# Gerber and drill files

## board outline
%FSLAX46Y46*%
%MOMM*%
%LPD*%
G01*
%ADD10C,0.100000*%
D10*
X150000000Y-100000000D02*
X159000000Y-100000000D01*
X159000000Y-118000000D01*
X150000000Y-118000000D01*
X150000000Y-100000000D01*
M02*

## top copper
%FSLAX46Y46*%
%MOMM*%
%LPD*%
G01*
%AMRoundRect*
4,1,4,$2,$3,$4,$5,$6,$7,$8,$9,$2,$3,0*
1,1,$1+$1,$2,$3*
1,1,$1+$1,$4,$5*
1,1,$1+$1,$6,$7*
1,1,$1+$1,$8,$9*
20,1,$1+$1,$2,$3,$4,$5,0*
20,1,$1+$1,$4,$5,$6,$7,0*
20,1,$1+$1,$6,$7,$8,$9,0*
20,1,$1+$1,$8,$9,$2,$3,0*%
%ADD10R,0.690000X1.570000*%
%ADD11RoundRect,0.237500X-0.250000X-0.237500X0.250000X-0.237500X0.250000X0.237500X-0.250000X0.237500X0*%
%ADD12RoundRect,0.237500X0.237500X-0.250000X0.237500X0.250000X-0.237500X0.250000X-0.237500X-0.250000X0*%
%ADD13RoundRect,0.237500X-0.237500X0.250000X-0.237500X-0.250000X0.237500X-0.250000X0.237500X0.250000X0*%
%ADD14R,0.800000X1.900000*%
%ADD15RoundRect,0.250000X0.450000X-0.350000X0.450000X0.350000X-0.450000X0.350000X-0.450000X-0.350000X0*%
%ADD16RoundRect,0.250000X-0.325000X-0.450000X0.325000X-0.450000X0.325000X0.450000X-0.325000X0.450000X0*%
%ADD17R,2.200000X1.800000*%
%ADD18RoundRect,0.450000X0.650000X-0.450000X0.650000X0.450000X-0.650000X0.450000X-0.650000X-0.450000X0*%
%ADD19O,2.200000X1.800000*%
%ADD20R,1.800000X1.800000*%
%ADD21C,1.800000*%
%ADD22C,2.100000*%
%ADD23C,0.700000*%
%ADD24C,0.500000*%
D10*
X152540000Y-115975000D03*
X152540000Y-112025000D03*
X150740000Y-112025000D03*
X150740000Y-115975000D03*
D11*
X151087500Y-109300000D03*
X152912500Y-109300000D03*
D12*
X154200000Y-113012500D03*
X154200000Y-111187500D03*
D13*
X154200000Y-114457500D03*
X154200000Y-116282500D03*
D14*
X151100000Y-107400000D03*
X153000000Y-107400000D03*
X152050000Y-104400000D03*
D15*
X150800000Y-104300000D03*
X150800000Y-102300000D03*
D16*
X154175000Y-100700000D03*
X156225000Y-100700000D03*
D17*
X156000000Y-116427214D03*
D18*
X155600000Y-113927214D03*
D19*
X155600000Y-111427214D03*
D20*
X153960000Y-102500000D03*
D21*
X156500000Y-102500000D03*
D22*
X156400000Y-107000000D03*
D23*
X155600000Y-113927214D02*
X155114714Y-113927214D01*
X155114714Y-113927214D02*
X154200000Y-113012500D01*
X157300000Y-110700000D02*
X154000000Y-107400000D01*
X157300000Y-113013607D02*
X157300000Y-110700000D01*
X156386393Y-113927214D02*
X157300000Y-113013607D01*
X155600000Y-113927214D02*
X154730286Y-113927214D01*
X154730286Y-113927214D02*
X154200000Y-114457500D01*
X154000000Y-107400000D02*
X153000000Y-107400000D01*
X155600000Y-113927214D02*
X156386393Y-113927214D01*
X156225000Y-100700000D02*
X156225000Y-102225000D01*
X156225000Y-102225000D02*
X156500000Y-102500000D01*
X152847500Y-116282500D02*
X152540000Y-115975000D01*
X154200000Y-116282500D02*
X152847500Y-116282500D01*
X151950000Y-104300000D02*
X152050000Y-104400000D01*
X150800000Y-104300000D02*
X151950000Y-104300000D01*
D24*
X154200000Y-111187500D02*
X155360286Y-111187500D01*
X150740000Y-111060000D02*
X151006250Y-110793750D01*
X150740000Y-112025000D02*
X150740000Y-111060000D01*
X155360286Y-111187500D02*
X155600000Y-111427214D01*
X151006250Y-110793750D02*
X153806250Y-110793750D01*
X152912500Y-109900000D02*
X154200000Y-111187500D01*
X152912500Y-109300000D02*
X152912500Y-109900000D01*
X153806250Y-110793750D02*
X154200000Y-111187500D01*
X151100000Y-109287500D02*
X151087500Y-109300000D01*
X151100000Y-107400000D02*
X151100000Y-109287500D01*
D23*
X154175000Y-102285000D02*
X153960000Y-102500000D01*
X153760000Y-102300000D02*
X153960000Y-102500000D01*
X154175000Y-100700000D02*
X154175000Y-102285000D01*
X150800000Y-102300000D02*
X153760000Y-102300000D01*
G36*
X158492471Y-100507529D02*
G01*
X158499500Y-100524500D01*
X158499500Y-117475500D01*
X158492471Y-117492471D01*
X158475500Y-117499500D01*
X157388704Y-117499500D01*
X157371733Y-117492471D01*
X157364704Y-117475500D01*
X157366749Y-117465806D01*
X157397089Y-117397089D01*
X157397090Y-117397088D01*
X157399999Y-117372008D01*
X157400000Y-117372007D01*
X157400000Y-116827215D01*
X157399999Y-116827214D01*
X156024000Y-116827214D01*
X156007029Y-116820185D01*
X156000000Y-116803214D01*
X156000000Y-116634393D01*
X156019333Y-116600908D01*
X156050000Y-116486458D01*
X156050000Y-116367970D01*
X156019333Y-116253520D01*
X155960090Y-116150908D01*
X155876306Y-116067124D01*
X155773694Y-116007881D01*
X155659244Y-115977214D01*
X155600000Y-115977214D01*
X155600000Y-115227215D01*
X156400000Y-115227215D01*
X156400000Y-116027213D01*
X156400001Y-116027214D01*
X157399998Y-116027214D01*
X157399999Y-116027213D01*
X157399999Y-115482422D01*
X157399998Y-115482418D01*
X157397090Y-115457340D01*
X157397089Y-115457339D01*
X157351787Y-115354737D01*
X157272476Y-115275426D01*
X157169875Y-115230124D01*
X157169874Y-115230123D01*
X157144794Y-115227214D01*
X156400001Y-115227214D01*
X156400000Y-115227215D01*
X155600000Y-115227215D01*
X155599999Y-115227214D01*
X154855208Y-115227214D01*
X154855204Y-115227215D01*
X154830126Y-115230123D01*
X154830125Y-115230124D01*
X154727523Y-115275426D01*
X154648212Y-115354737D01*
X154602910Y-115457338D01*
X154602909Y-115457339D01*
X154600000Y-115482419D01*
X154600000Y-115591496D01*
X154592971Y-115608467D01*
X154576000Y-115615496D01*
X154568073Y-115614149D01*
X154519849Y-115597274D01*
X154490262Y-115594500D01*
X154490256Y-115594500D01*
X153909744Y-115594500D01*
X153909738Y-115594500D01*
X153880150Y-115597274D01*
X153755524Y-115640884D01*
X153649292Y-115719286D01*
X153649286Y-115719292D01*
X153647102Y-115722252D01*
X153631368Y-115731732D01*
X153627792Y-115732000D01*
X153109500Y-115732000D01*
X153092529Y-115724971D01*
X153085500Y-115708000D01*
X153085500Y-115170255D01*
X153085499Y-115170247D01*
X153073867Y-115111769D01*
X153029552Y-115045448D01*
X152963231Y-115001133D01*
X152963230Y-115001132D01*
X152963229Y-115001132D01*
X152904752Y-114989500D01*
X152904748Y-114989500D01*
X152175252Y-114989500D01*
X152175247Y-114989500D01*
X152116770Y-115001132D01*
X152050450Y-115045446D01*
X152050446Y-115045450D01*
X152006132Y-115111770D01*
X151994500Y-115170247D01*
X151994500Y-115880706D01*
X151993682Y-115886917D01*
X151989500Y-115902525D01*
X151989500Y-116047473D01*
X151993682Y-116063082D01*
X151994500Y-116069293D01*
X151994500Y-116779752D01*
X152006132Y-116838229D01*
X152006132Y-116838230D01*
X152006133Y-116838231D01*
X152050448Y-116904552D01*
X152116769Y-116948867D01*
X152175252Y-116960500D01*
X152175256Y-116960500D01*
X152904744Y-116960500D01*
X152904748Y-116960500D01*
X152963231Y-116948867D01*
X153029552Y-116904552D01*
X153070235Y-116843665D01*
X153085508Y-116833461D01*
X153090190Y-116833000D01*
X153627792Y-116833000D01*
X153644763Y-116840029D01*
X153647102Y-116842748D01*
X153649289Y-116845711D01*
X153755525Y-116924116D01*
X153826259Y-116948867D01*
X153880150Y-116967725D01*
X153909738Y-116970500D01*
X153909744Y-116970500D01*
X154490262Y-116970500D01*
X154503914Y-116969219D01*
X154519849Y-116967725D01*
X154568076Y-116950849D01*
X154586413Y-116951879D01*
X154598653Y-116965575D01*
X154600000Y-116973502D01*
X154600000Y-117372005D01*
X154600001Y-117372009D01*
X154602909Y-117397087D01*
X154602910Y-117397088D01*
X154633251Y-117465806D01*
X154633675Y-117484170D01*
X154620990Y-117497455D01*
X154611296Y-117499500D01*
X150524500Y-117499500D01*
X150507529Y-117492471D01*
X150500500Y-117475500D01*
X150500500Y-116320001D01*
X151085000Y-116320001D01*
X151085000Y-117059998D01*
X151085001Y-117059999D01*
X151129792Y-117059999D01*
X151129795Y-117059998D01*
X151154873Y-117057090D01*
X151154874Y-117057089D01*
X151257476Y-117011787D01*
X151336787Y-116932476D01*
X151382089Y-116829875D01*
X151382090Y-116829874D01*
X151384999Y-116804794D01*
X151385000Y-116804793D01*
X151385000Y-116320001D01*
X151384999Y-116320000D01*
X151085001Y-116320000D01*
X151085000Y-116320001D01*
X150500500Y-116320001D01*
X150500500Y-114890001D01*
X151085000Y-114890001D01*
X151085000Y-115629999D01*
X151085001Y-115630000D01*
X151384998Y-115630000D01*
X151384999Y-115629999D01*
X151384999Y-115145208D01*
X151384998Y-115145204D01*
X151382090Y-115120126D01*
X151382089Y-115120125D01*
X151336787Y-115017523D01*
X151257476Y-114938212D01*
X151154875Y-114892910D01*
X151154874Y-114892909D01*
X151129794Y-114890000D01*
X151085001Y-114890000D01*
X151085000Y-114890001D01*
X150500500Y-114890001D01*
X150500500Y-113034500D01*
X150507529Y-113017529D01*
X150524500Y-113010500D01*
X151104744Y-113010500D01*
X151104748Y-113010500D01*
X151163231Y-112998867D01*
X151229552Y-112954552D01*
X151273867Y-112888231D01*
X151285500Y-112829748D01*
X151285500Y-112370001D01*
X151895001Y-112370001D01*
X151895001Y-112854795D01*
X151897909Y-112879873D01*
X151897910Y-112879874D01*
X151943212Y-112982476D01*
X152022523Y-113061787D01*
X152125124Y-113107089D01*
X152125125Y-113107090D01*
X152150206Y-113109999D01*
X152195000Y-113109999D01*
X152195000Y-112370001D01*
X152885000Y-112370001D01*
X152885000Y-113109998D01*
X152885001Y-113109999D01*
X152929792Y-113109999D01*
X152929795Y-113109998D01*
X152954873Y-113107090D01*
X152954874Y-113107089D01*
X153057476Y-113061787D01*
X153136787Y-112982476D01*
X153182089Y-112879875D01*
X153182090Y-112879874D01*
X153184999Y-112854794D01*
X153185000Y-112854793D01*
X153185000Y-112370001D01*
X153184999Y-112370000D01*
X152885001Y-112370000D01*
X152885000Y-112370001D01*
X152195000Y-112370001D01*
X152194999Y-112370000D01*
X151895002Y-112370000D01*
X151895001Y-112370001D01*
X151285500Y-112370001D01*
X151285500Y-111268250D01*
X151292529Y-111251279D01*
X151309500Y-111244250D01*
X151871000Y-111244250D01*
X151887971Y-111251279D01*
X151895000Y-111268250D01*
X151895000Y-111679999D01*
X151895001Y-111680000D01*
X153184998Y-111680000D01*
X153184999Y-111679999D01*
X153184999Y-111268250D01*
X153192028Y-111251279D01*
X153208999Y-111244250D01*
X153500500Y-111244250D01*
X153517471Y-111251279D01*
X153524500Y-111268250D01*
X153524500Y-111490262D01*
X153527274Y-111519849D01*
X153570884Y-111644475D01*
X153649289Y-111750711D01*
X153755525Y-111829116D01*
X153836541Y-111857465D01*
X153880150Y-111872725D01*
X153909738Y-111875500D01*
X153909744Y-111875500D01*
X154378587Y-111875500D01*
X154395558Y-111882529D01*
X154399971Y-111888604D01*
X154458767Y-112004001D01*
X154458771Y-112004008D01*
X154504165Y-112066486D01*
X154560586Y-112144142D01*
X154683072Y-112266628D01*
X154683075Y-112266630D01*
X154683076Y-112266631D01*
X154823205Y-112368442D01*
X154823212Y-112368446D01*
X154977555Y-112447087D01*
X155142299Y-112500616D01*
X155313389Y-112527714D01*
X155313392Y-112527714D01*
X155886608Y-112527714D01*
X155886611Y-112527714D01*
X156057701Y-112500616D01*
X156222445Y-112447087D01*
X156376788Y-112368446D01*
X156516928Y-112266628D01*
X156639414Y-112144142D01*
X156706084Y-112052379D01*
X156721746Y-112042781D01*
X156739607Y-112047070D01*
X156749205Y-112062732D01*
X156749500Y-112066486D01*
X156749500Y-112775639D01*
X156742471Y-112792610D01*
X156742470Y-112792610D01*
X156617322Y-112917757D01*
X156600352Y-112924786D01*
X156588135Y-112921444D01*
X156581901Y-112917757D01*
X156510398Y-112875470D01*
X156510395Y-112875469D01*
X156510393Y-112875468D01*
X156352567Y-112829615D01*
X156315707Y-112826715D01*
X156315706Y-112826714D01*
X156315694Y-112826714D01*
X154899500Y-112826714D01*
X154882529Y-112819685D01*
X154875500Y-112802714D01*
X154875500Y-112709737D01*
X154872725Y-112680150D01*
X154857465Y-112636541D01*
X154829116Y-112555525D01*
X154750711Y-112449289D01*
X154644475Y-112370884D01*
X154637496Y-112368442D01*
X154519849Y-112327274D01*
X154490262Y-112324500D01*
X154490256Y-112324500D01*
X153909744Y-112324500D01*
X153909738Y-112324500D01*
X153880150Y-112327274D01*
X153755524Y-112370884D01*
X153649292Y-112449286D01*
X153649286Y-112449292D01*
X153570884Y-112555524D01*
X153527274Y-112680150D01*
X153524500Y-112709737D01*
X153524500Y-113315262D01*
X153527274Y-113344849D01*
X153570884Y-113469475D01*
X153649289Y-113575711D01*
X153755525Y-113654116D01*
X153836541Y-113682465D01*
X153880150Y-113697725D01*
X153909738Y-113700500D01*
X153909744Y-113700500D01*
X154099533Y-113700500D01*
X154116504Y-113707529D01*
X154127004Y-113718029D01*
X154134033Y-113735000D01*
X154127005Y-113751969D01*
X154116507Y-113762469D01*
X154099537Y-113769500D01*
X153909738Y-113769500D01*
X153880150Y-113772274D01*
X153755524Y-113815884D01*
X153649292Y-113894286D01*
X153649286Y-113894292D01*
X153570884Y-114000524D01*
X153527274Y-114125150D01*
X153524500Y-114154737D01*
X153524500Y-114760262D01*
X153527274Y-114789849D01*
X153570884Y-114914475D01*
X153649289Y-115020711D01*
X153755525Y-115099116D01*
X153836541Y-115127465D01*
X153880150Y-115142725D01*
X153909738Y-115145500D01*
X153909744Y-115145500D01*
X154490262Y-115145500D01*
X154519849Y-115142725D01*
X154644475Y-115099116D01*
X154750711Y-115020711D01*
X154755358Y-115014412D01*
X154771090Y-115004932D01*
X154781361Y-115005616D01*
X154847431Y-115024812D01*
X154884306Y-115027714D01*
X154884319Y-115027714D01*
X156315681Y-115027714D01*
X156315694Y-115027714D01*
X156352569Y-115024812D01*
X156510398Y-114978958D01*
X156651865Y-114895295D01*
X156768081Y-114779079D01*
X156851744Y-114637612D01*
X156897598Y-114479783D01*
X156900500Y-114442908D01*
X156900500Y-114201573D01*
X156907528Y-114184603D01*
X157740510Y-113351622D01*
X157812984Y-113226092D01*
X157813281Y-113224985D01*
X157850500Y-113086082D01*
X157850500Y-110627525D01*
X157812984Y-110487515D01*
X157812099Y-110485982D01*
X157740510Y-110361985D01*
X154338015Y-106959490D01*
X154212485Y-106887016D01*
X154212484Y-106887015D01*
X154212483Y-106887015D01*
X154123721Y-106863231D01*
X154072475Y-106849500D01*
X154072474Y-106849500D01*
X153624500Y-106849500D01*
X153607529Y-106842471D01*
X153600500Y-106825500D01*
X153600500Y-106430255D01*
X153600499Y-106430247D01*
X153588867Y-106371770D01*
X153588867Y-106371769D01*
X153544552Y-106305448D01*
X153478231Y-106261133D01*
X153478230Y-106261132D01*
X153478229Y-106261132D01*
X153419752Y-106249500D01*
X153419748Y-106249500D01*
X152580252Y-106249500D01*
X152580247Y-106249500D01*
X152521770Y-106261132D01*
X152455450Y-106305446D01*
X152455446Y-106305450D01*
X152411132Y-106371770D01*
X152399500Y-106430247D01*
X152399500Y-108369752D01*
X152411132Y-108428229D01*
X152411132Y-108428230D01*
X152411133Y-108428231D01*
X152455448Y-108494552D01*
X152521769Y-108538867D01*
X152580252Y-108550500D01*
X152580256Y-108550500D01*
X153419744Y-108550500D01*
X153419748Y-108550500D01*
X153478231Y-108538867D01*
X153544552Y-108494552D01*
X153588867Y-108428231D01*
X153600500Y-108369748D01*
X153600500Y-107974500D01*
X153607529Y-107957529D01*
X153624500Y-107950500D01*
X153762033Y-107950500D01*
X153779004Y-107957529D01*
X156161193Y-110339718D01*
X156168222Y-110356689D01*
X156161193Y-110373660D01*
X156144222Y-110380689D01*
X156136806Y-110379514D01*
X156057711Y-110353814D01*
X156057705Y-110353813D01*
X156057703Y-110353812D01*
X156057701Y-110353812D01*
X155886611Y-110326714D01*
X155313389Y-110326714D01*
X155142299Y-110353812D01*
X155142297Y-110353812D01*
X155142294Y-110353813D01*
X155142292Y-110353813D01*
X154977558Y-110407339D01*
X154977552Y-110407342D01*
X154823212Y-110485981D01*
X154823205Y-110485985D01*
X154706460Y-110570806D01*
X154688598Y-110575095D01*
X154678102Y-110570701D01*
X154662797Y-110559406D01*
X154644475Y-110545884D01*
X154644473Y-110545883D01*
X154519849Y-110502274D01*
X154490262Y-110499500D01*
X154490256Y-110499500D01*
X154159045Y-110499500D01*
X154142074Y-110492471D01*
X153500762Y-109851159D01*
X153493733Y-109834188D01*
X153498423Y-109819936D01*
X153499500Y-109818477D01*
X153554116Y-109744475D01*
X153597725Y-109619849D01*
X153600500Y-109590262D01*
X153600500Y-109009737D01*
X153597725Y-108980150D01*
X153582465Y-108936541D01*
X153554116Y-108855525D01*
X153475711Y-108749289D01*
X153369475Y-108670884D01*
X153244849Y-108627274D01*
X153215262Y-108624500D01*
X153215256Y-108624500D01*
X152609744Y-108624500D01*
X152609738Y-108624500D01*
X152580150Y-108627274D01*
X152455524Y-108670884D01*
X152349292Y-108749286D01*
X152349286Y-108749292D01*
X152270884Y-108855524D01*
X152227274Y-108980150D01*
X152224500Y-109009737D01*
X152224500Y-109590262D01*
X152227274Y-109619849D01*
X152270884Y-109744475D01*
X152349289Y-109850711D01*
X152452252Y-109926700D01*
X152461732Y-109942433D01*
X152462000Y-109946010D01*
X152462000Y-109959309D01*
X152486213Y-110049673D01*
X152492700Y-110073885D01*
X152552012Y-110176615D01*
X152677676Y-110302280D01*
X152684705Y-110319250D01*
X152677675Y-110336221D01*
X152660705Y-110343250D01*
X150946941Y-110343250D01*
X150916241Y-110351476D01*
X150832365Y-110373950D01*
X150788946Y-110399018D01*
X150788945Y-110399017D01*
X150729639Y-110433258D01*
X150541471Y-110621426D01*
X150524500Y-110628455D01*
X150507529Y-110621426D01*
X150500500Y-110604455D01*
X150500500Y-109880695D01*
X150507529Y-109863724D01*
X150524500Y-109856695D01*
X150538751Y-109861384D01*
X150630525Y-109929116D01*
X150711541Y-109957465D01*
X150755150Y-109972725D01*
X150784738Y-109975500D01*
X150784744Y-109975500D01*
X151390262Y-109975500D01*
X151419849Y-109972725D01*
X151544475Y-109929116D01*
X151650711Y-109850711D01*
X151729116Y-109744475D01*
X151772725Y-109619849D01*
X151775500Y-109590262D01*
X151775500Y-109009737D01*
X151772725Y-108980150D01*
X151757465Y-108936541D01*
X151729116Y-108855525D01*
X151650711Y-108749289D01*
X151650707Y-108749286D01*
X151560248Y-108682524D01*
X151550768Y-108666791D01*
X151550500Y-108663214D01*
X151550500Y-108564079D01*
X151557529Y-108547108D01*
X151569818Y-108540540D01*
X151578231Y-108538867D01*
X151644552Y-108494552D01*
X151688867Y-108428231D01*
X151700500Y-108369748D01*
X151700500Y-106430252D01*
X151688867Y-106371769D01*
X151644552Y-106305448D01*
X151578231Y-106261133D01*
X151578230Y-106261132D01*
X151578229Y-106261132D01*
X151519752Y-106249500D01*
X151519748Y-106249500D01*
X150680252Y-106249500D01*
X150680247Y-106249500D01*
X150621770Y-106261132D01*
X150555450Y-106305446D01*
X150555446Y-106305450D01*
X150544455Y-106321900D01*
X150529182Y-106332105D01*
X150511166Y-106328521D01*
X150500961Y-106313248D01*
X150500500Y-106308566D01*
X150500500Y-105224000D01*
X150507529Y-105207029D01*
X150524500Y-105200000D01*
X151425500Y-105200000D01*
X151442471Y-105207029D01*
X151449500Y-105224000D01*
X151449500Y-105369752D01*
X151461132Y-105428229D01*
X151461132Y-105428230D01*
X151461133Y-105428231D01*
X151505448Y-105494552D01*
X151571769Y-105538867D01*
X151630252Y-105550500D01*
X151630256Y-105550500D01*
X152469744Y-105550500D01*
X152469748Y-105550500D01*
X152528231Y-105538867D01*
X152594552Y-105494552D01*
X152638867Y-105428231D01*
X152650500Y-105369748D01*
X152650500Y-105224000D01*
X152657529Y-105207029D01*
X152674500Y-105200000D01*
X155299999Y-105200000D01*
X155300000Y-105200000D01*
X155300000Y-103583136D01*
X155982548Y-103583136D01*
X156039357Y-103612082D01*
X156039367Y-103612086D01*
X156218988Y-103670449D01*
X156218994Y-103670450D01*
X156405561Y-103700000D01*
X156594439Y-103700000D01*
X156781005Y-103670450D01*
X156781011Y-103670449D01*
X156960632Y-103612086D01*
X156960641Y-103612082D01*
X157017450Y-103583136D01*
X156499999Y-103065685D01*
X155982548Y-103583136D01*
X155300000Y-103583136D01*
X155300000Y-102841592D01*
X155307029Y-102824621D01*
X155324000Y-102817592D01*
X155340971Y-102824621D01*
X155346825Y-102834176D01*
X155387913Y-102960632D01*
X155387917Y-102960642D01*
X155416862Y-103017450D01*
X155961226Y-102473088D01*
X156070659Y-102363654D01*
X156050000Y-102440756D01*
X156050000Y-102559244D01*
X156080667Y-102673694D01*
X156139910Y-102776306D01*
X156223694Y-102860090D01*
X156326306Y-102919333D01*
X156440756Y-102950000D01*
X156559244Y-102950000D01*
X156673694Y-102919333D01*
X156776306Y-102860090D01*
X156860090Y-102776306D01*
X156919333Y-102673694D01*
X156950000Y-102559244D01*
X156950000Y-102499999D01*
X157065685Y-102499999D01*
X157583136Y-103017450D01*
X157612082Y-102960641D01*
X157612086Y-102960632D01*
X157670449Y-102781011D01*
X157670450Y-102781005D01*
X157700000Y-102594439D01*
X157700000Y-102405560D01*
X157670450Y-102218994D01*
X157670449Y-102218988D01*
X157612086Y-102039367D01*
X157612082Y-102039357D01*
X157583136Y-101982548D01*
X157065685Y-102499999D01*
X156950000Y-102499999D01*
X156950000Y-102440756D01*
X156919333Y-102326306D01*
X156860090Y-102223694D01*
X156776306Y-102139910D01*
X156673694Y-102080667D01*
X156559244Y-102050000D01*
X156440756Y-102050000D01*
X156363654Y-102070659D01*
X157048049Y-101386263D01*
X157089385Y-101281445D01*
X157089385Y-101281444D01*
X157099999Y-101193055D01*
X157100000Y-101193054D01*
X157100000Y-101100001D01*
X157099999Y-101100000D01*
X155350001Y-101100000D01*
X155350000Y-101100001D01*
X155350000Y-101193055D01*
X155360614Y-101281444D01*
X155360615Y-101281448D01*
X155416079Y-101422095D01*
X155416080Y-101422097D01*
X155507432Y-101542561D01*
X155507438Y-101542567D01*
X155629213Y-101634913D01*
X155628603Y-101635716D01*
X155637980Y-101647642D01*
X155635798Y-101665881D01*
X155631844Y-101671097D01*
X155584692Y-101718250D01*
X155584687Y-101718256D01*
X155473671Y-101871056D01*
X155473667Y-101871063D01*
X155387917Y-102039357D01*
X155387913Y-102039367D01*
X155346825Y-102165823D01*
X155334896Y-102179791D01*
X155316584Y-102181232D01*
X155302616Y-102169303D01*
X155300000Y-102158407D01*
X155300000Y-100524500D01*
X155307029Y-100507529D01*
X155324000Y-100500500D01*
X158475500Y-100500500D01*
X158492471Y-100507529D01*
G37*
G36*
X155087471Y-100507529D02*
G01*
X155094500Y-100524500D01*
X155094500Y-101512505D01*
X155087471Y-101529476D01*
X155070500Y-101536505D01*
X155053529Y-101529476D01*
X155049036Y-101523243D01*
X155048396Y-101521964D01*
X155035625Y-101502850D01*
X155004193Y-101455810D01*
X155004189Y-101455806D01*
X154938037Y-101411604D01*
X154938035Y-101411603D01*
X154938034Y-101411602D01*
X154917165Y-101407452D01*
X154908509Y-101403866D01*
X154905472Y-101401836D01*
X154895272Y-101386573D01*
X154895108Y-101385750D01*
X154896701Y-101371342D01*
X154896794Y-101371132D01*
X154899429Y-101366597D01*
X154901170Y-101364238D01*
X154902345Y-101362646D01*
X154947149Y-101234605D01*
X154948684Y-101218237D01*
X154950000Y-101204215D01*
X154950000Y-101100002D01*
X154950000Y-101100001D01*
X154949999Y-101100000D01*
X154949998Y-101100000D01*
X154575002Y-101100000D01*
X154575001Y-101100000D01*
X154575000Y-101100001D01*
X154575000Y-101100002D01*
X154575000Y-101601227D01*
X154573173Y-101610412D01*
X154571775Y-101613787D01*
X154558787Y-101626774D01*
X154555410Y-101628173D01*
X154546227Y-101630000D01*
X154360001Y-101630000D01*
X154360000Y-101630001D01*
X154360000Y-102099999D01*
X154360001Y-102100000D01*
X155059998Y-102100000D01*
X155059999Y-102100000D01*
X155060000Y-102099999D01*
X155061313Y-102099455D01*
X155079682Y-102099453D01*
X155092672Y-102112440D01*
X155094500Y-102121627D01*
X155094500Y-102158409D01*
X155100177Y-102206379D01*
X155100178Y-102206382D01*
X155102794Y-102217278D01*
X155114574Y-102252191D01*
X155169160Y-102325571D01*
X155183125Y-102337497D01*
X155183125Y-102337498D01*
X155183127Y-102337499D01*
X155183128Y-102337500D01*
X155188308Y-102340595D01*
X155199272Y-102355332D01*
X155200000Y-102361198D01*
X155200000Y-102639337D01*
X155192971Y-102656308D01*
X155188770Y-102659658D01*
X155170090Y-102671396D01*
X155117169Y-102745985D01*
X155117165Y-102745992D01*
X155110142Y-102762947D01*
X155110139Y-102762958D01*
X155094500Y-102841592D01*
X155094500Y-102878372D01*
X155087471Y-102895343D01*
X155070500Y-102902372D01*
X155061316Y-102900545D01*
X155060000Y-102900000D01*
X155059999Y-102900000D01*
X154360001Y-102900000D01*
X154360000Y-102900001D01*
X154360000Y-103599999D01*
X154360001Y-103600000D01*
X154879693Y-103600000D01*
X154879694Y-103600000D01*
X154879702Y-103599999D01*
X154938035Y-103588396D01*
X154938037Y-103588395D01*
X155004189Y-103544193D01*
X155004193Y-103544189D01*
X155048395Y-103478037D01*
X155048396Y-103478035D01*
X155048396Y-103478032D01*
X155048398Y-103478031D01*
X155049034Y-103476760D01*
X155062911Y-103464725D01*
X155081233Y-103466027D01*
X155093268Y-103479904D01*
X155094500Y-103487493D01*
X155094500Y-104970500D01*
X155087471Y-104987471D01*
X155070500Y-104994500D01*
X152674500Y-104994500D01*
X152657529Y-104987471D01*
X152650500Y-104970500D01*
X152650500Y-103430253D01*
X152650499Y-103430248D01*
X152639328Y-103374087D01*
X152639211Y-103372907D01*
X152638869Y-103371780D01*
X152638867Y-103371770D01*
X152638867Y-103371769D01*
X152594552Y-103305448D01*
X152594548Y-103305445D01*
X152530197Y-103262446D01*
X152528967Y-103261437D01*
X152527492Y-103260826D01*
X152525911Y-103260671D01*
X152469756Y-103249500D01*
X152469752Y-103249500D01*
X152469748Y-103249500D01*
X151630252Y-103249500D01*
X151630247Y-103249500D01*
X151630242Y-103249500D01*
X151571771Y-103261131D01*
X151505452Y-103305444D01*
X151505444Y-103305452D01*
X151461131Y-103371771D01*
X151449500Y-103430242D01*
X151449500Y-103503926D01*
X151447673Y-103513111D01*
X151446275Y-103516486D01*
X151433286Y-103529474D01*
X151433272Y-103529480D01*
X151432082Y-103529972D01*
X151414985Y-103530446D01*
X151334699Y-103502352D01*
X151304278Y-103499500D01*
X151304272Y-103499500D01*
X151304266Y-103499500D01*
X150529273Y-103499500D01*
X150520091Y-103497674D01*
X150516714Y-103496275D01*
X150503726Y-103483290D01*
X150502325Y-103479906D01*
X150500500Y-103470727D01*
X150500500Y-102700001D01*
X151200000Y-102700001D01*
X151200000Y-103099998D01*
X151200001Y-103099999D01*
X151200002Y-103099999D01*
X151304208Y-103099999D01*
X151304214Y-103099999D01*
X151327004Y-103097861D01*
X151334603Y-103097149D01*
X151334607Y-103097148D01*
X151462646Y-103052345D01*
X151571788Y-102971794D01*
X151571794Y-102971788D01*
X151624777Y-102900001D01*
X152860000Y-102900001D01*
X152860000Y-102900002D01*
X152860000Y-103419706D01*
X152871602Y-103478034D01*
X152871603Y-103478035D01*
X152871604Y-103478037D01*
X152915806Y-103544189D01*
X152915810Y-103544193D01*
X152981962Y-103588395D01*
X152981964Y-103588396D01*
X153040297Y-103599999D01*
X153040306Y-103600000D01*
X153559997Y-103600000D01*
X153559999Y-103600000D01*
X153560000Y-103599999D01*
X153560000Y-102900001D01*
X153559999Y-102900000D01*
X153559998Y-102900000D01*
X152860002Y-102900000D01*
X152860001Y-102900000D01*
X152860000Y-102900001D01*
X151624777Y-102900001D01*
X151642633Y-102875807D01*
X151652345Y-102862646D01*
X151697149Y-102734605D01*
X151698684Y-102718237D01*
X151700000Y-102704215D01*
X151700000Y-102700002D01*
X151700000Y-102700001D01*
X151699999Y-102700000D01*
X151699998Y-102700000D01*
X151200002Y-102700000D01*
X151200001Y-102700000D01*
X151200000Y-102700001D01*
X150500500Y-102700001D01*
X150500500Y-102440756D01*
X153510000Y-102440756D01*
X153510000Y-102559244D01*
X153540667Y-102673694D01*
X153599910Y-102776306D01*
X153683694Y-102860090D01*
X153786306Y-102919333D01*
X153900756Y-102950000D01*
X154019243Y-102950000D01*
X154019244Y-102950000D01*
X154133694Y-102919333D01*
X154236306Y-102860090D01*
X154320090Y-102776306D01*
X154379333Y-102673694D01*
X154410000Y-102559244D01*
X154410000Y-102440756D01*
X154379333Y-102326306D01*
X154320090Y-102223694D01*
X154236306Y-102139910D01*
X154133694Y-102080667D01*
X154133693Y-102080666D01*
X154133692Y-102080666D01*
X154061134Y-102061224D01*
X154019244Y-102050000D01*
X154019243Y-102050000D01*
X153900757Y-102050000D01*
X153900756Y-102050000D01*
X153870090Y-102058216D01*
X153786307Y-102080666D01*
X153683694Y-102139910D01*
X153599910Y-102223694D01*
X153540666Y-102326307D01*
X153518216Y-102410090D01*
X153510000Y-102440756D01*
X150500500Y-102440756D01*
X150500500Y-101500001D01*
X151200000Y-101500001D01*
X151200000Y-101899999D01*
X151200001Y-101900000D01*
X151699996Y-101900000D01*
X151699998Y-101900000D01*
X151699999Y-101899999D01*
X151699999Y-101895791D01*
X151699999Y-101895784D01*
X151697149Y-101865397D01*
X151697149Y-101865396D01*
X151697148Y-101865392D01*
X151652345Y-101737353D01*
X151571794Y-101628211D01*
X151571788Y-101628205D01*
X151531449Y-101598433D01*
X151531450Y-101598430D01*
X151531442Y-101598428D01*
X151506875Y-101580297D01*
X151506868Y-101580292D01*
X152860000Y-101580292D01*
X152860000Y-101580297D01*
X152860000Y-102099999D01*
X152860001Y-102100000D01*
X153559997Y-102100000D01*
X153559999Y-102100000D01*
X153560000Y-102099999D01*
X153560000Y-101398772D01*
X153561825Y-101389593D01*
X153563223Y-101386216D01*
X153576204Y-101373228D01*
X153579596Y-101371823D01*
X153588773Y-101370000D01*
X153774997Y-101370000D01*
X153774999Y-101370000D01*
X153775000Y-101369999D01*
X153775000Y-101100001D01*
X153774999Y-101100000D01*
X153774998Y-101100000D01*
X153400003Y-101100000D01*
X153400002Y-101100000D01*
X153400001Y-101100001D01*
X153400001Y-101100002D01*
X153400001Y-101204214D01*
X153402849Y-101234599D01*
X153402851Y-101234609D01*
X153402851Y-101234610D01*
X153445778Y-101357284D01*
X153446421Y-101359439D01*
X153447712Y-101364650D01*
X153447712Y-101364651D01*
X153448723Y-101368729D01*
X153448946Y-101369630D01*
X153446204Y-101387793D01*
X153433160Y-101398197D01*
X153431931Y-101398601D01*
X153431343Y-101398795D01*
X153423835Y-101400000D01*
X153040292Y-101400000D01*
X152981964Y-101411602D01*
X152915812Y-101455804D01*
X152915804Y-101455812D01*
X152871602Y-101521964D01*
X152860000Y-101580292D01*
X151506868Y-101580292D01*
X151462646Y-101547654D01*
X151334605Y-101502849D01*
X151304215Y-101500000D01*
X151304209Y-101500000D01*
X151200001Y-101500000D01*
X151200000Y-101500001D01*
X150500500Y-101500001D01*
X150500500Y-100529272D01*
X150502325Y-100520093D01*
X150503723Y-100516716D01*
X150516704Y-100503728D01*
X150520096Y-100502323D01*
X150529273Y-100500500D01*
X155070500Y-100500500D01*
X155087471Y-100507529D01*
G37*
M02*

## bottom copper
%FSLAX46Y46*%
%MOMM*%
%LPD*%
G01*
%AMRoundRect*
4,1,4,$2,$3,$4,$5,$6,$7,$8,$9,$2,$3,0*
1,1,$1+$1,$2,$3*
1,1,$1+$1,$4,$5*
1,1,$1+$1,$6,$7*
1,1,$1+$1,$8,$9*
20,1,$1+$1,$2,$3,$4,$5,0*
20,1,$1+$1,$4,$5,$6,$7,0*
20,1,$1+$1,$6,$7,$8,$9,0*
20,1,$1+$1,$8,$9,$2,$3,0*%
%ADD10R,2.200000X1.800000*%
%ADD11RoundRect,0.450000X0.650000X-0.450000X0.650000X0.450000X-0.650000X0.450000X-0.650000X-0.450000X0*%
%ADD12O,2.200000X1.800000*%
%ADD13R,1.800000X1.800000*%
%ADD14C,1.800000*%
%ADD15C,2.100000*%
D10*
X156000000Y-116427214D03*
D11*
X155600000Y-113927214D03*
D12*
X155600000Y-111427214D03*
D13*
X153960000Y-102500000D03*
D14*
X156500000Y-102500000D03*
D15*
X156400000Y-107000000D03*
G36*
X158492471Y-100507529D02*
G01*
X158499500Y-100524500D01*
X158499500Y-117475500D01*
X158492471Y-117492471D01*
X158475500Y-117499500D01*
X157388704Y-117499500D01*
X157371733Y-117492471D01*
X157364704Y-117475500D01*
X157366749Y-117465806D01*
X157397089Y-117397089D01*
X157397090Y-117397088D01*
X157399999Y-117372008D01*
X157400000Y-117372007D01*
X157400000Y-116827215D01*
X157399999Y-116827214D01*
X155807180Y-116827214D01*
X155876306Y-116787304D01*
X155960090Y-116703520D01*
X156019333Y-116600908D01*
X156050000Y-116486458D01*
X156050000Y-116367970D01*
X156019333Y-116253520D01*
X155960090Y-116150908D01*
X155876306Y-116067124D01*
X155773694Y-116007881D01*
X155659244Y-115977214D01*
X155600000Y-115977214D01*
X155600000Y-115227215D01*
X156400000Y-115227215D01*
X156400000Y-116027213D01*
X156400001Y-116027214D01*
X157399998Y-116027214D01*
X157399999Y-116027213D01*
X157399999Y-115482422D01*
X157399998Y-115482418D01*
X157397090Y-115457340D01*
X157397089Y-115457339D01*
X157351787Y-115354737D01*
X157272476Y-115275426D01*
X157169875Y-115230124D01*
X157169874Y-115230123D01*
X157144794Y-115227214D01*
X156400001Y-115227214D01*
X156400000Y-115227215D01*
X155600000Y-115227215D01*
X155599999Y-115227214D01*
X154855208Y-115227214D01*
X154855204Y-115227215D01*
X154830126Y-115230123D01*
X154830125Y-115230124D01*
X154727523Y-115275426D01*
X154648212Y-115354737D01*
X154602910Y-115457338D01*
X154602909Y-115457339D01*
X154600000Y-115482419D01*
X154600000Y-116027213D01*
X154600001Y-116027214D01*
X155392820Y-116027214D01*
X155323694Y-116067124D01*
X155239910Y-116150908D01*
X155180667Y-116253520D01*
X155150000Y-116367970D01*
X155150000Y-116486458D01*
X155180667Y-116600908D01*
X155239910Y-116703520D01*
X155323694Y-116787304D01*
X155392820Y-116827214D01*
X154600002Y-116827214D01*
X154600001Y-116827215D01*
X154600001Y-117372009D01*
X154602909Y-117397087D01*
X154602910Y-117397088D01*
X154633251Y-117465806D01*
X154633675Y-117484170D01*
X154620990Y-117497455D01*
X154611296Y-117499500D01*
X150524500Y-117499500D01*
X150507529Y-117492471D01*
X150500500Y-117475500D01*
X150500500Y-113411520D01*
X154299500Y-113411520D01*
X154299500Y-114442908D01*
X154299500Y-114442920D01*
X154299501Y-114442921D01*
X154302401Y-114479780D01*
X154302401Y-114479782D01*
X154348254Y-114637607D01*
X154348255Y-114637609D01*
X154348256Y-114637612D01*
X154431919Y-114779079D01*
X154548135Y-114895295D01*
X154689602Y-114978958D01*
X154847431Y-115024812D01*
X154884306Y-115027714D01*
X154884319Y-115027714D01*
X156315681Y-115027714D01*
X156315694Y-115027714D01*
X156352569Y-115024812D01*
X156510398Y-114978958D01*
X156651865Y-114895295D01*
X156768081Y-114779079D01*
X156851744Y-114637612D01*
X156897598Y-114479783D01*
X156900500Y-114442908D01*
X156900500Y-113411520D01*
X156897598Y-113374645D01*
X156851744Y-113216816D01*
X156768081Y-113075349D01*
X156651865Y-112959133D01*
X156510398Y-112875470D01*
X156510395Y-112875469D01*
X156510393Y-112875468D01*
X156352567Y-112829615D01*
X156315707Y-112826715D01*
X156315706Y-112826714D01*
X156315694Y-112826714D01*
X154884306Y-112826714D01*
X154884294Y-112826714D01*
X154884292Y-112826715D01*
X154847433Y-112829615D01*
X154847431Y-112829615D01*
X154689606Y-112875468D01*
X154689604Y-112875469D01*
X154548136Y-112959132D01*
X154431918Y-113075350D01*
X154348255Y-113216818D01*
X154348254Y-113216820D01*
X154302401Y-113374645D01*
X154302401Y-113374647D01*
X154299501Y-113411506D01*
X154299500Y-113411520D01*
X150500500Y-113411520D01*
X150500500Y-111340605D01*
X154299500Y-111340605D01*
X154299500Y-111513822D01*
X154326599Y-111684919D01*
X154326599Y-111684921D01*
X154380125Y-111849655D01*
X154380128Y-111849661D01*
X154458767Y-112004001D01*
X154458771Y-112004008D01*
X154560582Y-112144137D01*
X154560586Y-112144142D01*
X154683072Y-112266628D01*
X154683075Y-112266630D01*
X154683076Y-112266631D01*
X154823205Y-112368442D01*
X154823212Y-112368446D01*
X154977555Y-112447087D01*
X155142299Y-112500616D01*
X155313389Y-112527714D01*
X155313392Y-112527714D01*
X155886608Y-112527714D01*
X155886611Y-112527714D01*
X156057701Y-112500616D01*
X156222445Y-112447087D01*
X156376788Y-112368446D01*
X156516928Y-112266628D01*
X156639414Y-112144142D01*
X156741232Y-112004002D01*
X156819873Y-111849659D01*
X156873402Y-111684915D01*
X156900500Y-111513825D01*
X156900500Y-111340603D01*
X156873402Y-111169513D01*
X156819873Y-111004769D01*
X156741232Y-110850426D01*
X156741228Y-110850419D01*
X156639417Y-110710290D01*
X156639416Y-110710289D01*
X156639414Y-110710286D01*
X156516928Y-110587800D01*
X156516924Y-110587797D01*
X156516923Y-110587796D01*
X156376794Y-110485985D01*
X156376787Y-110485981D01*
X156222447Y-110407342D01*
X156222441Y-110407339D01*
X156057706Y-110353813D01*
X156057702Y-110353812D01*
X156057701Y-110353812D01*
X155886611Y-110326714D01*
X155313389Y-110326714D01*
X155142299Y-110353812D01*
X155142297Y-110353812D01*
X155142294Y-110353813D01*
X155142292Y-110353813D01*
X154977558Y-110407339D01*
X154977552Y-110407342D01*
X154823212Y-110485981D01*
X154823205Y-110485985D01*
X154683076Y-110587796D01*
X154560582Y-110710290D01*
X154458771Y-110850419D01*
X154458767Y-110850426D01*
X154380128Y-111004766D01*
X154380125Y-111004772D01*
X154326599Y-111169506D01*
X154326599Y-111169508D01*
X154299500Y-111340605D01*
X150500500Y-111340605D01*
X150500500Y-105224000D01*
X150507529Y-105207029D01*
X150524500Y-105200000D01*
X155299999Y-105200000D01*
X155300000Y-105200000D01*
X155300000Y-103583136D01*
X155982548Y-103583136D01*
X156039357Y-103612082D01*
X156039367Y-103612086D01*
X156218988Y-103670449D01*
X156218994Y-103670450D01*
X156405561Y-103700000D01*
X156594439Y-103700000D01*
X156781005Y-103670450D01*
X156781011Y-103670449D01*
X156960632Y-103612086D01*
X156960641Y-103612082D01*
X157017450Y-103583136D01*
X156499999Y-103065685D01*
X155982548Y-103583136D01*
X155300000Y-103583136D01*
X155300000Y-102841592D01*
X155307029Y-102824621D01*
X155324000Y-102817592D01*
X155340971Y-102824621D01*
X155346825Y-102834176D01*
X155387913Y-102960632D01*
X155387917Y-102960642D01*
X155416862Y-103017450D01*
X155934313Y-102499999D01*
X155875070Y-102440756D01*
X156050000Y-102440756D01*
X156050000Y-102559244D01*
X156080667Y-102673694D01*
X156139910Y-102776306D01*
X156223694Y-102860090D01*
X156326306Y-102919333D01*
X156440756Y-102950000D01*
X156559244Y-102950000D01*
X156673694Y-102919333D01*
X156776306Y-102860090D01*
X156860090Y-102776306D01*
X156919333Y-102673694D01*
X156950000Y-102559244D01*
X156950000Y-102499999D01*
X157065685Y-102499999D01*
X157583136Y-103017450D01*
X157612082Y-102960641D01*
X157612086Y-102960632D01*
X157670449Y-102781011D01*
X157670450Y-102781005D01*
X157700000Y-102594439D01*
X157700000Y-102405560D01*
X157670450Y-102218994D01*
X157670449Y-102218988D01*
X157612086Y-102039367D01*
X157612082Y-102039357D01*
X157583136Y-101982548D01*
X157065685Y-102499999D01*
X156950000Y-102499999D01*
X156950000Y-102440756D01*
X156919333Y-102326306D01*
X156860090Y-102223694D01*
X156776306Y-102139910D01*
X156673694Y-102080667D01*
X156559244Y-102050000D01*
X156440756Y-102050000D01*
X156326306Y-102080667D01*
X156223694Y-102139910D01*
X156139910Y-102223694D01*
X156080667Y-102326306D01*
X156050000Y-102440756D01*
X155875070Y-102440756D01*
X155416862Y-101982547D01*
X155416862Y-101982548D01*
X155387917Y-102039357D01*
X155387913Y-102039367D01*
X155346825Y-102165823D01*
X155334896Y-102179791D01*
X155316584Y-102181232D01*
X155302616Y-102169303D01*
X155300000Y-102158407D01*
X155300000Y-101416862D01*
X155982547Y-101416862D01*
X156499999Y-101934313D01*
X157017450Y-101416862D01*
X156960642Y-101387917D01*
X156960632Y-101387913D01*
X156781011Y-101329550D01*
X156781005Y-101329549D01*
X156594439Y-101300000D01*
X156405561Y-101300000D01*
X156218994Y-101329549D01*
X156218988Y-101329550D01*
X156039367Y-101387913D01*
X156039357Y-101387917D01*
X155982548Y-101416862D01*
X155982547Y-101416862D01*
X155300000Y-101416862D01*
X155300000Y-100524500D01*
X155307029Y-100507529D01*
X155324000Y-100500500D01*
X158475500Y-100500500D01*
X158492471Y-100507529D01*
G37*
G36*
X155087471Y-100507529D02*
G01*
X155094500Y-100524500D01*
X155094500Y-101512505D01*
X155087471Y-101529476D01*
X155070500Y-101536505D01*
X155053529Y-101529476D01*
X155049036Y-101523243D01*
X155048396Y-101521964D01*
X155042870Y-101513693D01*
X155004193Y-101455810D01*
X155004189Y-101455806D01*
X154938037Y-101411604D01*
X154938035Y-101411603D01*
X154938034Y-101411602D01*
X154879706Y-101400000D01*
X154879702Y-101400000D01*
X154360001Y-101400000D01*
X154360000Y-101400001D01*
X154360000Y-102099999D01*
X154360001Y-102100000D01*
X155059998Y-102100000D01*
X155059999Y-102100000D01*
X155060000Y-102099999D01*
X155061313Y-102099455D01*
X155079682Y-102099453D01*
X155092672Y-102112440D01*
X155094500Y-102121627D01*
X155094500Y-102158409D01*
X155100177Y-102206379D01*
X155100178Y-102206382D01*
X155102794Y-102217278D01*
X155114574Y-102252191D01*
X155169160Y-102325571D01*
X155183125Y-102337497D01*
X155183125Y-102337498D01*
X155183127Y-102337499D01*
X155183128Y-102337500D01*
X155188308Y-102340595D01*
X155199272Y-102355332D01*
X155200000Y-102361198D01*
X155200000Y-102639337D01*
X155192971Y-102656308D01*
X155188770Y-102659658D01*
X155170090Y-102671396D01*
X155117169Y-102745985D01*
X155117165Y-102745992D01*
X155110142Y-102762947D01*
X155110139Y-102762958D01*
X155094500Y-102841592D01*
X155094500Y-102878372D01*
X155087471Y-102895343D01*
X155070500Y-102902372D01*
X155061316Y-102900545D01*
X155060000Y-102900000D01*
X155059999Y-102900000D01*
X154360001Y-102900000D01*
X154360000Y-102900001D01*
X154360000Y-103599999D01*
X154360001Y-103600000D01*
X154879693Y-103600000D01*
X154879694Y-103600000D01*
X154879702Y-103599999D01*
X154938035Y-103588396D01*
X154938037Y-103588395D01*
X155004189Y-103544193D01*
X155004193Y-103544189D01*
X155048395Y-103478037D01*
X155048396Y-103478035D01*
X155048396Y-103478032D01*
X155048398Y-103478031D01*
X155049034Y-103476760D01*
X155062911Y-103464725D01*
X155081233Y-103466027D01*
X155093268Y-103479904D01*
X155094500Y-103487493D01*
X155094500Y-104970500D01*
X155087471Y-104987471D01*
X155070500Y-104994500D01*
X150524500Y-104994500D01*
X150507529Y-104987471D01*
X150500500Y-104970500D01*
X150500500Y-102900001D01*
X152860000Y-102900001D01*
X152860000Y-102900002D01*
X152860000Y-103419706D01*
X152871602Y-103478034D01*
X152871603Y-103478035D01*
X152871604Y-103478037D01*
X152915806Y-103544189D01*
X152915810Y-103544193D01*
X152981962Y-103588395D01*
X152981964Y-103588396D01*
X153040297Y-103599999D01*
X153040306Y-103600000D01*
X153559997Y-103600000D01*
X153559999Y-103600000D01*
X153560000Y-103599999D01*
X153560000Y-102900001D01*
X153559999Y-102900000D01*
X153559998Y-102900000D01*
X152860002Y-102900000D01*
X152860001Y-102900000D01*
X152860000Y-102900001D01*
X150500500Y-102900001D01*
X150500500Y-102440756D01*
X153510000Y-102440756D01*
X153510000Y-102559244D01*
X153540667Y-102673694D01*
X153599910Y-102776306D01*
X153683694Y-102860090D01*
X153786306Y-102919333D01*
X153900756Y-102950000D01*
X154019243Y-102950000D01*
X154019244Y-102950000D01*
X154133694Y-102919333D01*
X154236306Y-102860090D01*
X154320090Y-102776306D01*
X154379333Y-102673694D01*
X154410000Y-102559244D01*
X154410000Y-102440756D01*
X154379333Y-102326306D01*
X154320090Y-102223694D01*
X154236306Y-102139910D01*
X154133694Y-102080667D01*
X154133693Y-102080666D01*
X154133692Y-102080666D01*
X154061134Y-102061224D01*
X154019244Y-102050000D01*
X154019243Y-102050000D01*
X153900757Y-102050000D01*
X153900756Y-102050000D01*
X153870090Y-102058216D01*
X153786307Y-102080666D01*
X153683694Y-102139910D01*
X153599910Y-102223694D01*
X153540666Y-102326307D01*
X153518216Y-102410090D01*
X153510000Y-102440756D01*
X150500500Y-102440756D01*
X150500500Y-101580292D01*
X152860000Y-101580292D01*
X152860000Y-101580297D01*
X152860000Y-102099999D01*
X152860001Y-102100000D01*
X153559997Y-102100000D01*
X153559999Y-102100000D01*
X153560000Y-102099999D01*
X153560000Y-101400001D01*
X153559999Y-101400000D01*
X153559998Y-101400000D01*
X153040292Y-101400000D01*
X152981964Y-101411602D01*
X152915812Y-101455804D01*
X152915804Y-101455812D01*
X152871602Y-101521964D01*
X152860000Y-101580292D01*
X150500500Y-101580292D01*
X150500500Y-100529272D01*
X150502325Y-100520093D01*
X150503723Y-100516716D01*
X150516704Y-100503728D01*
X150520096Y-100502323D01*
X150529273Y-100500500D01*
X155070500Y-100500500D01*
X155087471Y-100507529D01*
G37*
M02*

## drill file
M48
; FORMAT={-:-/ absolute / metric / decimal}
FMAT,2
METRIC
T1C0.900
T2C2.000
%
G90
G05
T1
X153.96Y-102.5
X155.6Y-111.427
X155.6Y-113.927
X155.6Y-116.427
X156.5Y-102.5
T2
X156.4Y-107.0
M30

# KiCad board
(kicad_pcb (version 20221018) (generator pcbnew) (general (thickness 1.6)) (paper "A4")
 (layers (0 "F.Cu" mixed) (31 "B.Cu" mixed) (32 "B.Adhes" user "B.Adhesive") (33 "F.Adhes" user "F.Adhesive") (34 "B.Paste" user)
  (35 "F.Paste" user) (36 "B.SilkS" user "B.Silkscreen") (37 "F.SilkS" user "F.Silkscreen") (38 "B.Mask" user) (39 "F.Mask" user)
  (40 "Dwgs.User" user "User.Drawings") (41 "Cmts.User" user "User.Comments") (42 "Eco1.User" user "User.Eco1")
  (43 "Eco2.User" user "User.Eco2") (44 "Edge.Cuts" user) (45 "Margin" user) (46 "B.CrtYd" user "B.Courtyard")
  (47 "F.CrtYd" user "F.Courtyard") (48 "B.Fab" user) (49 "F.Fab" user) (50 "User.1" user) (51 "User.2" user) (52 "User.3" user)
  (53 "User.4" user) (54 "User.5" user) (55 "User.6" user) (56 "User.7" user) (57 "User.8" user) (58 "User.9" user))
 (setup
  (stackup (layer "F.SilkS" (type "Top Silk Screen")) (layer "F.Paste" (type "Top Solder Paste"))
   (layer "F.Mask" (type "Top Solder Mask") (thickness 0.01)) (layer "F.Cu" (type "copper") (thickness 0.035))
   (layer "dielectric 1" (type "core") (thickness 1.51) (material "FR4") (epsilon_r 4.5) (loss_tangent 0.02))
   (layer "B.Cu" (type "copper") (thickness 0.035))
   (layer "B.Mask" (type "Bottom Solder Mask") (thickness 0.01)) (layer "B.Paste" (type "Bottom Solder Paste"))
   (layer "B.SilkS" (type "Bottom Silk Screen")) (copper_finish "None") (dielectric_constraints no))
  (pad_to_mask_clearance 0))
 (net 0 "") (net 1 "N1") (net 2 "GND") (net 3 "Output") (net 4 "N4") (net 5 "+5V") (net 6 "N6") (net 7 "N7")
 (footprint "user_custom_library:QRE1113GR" (layer "F.Cu") (at 151.64 114 180)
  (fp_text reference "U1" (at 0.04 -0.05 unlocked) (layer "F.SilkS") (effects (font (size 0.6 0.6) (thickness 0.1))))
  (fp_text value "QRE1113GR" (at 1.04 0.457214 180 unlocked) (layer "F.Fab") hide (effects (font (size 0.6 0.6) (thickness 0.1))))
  (pad "1" smd rect (at -0.9 -1.975 180) (size 0.69 1.57) (layers "F.Cu" "F.Paste" "F.Mask") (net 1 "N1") (solder_mask_margin 0.102))
  (pad "2" smd rect (at -0.9 1.975 180) (size 0.69 1.57) (layers "F.Cu" "F.Paste" "F.Mask") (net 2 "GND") (solder_mask_margin 0.102))
  (pad "3" smd rect (at 0.9 1.975 180) (size 0.69 1.57) (layers "F.Cu" "F.Paste" "F.Mask") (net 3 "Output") (solder_mask_margin 0.102))
  (pad "4" smd rect (at 0.9 -1.975 180) (size 0.69 1.57) (layers "F.Cu" "F.Paste" "F.Mask") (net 2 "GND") (solder_mask_margin 0.102)))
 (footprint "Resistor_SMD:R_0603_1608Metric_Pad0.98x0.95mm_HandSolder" (layer "F.Cu") (at 152 109.3)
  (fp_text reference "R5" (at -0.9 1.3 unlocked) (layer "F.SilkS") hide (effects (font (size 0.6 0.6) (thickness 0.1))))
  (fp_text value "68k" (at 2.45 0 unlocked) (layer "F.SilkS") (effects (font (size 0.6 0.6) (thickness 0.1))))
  (pad "1" smd roundrect (at -0.9125 0) (size 0.975 0.95) (layers "F.Cu" "F.Paste" "F.Mask") (roundrect_rratio 0.25) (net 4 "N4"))
  (pad "2" smd roundrect (at 0.9125 0) (size 0.975 0.95) (layers "F.Cu" "F.Paste" "F.Mask") (roundrect_rratio 0.25) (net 3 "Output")))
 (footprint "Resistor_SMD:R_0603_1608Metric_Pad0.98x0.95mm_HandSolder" (layer "F.Cu") (at 154.2 112.1 90)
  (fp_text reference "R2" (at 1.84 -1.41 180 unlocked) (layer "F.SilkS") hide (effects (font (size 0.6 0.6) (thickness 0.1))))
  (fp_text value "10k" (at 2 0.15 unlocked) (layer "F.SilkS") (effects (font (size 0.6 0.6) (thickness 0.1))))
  (pad "1" smd roundrect (at -0.9125 0 90) (size 0.975 0.95) (layers "F.Cu" "F.Paste" "F.Mask") (roundrect_rratio 0.25) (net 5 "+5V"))
  (pad "2" smd roundrect (at 0.9125 0 90) (size 0.975 0.95) (layers "F.Cu" "F.Paste" "F.Mask") (roundrect_rratio 0.25) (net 3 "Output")))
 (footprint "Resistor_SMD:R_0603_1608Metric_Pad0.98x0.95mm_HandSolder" (layer "F.Cu") (at 154.2 115.37 -90)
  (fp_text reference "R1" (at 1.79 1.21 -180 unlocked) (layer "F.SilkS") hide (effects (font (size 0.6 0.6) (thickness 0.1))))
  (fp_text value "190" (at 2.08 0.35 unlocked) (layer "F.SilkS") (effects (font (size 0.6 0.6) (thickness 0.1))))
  (pad "1" smd roundrect (at -0.9125 0 270) (size 0.975 0.95) (layers "F.Cu" "F.Paste" "F.Mask") (roundrect_rratio 0.25) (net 5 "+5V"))
  (pad "2" smd roundrect (at 0.9125 0 270) (size 0.975 0.95) (layers "F.Cu" "F.Paste" "F.Mask") (roundrect_rratio 0.25) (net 1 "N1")))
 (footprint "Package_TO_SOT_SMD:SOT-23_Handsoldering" (layer "F.Cu") (at 152.05 105.9 90)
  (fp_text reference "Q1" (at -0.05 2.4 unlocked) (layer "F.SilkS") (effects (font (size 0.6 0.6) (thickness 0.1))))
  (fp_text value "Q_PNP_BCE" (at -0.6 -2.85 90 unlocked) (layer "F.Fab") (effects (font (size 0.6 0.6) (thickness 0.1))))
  (pad "1" smd rect (at -1.5 -0.95 90) (size 1.9 0.8) (layers "F.Cu" "F.Paste" "F.Mask") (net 4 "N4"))
  (pad "2" smd rect (at -1.5 0.95 90) (size 1.9 0.8) (layers "F.Cu" "F.Paste" "F.Mask") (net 5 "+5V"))
  (pad "3" smd rect (at 1.5 0 90) (size 1.9 0.8) (layers "F.Cu" "F.Paste" "F.Mask") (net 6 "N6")))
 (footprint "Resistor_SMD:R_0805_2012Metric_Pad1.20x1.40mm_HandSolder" (layer "F.Cu") (at 150.8 103.3 90)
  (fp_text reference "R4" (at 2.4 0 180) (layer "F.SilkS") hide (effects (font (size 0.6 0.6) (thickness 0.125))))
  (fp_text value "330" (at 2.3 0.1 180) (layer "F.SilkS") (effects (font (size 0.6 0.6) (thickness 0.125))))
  (pad "1" smd roundrect (at -1 0 90) (size 1.2 1.4) (layers "F.Cu" "F.Paste" "F.Mask") (roundrect_rratio 0.2083333333) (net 6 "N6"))
  (pad "2" smd roundrect (at 1 0 90) (size 1.2 1.4) (layers "F.Cu" "F.Paste" "F.Mask") (roundrect_rratio 0.2083333333) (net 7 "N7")))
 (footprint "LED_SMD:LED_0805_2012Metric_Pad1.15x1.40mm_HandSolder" (layer "F.Cu") (at 155.2 100.7)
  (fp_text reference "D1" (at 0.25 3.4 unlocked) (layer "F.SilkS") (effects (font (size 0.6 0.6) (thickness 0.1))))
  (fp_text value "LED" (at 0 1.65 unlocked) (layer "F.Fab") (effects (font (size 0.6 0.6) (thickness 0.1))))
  (pad "1" smd roundrect (at -1.025 0) (size 1.15 1.4) (layers "F.Cu" "F.Paste" "F.Mask") (roundrect_rratio 0.2173913043) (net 7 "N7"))
  (pad "2" smd roundrect (at 1.025 0) (size 1.15 1.4) (layers "F.Cu" "F.Paste" "F.Mask") (roundrect_rratio 0.2173913043) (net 2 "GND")))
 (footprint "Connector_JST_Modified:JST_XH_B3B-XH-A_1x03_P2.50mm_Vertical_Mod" (layer "B.Cu") (at 155.6 116.427214 90)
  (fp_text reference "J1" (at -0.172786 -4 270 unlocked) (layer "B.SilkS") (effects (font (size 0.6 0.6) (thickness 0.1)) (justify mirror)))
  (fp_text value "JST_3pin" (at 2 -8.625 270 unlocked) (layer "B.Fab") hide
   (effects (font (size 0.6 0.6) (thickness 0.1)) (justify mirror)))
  (pad "1" thru_hole rect (at 0 0 90) (size 1.8 2.2) (drill 0.9 (offset 0 0.4)) (layers "*.Cu" "*.Mask") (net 2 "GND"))
  (pad "2" thru_hole roundrect (at 2.5 0 90) (size 1.8 2.2) (drill 0.9) (layers "*.Cu" "*.Mask") (roundrect_rratio 0.25) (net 5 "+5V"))
  (pad "3" thru_hole oval (at 5 0 90) (size 1.8 2.2) (drill 0.9) (layers "*.Cu" "*.Mask") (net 3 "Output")))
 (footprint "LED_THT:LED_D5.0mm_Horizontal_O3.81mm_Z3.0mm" (layer "B.Cu") (at 153.96 102.5)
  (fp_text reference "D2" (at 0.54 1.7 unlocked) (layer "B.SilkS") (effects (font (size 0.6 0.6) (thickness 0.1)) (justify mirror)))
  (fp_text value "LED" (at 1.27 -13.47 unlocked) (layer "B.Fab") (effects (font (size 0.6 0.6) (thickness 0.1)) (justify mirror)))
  (pad "1" thru_hole rect (at 0 0) (size 1.8 1.8) (drill 0.9) (layers "*.Cu" "*.Mask") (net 7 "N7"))
  (pad "2" thru_hole circle (at 2.54 0) (size 1.8 1.8) (drill 0.9) (layers "*.Cu" "*.Mask") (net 2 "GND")))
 (gr_rect locked (start 150 100) (end 159 118) (stroke (width 0.1) (type solid)) (fill none) (layer "Edge.Cuts"))
 (segment (start 155.6 113.927214) (end 155.114714 113.927214) (width 0.7) (layer "F.Cu") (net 5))
 (segment (start 155.114714 113.927214) (end 154.2 113.0125) (width 0.7) (layer "F.Cu") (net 5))
 (segment (start 157.3 110.7) (end 154 107.4) (width 0.7) (layer "F.Cu") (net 5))
 (segment (start 157.3 113.013607) (end 157.3 110.7) (width 0.7) (layer "F.Cu") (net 5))
 (segment (start 156.386393 113.927214) (end 157.3 113.013607) (width 0.7) (layer "F.Cu") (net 5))
 (segment (start 155.6 113.927214) (end 154.730286 113.927214) (width 0.7) (layer "F.Cu") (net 5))
 (segment (start 154.730286 113.927214) (end 154.2 114.4575) (width 0.7) (layer "F.Cu") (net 5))
 (segment (start 154 107.4) (end 153 107.4) (width 0.7) (layer "F.Cu") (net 5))
 (segment (start 155.6 113.927214) (end 156.386393 113.927214) (width 0.7) (layer "F.Cu") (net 5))
 (segment (start 156.225 100.7) (end 156.225 102.225) (width 0.7) (layer "F.Cu") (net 2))
 (segment (start 156.225 102.225) (end 156.5 102.5) (width 0.7) (layer "F.Cu") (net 2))
 (via (at 156.4 107) (size 2.1) (drill 2) (layers "F.Cu" "B.Cu") (free) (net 2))
 (segment (start 152.8475 116.2825) (end 152.54 115.975) (width 0.7) (layer "F.Cu") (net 1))
 (segment (start 154.2 116.2825) (end 152.8475 116.2825) (width 0.7) (layer "F.Cu") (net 1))
 (segment (start 151.95 104.3) (end 152.05 104.4) (width 0.7) (layer "F.Cu") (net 6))
 (segment (start 150.8 104.3) (end 151.95 104.3) (width 0.7) (layer "F.Cu") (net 6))
 (segment (start 154.2 111.1875) (end 155.360286 111.1875) (width 0.5) (layer "F.Cu") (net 3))
 (segment (start 150.74 111.06) (end 151.00625 110.79375) (width 0.5) (layer "F.Cu") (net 3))
 (segment (start 150.74 112.025) (end 150.74 111.06) (width 0.5) (layer "F.Cu") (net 3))
 (segment (start 155.360286 111.1875) (end 155.6 111.427214) (width 0.5) (layer "F.Cu") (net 3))
 (segment (start 151.00625 110.79375) (end 153.80625 110.79375) (width 0.5) (layer "F.Cu") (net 3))
 (segment (start 152.9125 109.9) (end 154.2 111.1875) (width 0.5) (layer "F.Cu") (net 3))
 (segment (start 152.9125 109.3) (end 152.9125 109.9) (width 0.5) (layer "F.Cu") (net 3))
 (segment (start 153.80625 110.79375) (end 154.2 111.1875) (width 0.5) (layer "F.Cu") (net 3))
 (segment (start 151.1 109.2875) (end 151.0875 109.3) (width 0.5) (layer "F.Cu") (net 4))
 (segment (start 151.1 107.4) (end 151.1 109.2875) (width 0.5) (layer "F.Cu") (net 4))
 (segment (start 154.175 102.285) (end 153.96 102.5) (width 0.7) (layer "F.Cu") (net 7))
 (segment (start 153.76 102.3) (end 153.96 102.5) (width 0.7) (layer "F.Cu") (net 7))
 (segment (start 154.175 100.7) (end 154.175 102.285) (width 0.7) (layer "F.Cu") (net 7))
 (segment (start 150.8 102.3) (end 153.76 102.3) (width 0.7) (layer "F.Cu") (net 7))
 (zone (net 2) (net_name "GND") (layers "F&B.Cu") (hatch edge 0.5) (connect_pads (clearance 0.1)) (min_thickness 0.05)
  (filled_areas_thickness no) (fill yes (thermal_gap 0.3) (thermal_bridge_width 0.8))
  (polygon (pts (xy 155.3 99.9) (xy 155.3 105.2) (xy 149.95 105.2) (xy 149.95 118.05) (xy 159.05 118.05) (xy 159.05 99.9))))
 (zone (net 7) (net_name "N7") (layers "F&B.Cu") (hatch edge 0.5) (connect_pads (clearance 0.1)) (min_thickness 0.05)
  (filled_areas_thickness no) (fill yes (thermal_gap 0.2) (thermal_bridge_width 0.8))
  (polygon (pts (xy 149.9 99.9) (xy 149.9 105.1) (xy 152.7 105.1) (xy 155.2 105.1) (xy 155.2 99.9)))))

